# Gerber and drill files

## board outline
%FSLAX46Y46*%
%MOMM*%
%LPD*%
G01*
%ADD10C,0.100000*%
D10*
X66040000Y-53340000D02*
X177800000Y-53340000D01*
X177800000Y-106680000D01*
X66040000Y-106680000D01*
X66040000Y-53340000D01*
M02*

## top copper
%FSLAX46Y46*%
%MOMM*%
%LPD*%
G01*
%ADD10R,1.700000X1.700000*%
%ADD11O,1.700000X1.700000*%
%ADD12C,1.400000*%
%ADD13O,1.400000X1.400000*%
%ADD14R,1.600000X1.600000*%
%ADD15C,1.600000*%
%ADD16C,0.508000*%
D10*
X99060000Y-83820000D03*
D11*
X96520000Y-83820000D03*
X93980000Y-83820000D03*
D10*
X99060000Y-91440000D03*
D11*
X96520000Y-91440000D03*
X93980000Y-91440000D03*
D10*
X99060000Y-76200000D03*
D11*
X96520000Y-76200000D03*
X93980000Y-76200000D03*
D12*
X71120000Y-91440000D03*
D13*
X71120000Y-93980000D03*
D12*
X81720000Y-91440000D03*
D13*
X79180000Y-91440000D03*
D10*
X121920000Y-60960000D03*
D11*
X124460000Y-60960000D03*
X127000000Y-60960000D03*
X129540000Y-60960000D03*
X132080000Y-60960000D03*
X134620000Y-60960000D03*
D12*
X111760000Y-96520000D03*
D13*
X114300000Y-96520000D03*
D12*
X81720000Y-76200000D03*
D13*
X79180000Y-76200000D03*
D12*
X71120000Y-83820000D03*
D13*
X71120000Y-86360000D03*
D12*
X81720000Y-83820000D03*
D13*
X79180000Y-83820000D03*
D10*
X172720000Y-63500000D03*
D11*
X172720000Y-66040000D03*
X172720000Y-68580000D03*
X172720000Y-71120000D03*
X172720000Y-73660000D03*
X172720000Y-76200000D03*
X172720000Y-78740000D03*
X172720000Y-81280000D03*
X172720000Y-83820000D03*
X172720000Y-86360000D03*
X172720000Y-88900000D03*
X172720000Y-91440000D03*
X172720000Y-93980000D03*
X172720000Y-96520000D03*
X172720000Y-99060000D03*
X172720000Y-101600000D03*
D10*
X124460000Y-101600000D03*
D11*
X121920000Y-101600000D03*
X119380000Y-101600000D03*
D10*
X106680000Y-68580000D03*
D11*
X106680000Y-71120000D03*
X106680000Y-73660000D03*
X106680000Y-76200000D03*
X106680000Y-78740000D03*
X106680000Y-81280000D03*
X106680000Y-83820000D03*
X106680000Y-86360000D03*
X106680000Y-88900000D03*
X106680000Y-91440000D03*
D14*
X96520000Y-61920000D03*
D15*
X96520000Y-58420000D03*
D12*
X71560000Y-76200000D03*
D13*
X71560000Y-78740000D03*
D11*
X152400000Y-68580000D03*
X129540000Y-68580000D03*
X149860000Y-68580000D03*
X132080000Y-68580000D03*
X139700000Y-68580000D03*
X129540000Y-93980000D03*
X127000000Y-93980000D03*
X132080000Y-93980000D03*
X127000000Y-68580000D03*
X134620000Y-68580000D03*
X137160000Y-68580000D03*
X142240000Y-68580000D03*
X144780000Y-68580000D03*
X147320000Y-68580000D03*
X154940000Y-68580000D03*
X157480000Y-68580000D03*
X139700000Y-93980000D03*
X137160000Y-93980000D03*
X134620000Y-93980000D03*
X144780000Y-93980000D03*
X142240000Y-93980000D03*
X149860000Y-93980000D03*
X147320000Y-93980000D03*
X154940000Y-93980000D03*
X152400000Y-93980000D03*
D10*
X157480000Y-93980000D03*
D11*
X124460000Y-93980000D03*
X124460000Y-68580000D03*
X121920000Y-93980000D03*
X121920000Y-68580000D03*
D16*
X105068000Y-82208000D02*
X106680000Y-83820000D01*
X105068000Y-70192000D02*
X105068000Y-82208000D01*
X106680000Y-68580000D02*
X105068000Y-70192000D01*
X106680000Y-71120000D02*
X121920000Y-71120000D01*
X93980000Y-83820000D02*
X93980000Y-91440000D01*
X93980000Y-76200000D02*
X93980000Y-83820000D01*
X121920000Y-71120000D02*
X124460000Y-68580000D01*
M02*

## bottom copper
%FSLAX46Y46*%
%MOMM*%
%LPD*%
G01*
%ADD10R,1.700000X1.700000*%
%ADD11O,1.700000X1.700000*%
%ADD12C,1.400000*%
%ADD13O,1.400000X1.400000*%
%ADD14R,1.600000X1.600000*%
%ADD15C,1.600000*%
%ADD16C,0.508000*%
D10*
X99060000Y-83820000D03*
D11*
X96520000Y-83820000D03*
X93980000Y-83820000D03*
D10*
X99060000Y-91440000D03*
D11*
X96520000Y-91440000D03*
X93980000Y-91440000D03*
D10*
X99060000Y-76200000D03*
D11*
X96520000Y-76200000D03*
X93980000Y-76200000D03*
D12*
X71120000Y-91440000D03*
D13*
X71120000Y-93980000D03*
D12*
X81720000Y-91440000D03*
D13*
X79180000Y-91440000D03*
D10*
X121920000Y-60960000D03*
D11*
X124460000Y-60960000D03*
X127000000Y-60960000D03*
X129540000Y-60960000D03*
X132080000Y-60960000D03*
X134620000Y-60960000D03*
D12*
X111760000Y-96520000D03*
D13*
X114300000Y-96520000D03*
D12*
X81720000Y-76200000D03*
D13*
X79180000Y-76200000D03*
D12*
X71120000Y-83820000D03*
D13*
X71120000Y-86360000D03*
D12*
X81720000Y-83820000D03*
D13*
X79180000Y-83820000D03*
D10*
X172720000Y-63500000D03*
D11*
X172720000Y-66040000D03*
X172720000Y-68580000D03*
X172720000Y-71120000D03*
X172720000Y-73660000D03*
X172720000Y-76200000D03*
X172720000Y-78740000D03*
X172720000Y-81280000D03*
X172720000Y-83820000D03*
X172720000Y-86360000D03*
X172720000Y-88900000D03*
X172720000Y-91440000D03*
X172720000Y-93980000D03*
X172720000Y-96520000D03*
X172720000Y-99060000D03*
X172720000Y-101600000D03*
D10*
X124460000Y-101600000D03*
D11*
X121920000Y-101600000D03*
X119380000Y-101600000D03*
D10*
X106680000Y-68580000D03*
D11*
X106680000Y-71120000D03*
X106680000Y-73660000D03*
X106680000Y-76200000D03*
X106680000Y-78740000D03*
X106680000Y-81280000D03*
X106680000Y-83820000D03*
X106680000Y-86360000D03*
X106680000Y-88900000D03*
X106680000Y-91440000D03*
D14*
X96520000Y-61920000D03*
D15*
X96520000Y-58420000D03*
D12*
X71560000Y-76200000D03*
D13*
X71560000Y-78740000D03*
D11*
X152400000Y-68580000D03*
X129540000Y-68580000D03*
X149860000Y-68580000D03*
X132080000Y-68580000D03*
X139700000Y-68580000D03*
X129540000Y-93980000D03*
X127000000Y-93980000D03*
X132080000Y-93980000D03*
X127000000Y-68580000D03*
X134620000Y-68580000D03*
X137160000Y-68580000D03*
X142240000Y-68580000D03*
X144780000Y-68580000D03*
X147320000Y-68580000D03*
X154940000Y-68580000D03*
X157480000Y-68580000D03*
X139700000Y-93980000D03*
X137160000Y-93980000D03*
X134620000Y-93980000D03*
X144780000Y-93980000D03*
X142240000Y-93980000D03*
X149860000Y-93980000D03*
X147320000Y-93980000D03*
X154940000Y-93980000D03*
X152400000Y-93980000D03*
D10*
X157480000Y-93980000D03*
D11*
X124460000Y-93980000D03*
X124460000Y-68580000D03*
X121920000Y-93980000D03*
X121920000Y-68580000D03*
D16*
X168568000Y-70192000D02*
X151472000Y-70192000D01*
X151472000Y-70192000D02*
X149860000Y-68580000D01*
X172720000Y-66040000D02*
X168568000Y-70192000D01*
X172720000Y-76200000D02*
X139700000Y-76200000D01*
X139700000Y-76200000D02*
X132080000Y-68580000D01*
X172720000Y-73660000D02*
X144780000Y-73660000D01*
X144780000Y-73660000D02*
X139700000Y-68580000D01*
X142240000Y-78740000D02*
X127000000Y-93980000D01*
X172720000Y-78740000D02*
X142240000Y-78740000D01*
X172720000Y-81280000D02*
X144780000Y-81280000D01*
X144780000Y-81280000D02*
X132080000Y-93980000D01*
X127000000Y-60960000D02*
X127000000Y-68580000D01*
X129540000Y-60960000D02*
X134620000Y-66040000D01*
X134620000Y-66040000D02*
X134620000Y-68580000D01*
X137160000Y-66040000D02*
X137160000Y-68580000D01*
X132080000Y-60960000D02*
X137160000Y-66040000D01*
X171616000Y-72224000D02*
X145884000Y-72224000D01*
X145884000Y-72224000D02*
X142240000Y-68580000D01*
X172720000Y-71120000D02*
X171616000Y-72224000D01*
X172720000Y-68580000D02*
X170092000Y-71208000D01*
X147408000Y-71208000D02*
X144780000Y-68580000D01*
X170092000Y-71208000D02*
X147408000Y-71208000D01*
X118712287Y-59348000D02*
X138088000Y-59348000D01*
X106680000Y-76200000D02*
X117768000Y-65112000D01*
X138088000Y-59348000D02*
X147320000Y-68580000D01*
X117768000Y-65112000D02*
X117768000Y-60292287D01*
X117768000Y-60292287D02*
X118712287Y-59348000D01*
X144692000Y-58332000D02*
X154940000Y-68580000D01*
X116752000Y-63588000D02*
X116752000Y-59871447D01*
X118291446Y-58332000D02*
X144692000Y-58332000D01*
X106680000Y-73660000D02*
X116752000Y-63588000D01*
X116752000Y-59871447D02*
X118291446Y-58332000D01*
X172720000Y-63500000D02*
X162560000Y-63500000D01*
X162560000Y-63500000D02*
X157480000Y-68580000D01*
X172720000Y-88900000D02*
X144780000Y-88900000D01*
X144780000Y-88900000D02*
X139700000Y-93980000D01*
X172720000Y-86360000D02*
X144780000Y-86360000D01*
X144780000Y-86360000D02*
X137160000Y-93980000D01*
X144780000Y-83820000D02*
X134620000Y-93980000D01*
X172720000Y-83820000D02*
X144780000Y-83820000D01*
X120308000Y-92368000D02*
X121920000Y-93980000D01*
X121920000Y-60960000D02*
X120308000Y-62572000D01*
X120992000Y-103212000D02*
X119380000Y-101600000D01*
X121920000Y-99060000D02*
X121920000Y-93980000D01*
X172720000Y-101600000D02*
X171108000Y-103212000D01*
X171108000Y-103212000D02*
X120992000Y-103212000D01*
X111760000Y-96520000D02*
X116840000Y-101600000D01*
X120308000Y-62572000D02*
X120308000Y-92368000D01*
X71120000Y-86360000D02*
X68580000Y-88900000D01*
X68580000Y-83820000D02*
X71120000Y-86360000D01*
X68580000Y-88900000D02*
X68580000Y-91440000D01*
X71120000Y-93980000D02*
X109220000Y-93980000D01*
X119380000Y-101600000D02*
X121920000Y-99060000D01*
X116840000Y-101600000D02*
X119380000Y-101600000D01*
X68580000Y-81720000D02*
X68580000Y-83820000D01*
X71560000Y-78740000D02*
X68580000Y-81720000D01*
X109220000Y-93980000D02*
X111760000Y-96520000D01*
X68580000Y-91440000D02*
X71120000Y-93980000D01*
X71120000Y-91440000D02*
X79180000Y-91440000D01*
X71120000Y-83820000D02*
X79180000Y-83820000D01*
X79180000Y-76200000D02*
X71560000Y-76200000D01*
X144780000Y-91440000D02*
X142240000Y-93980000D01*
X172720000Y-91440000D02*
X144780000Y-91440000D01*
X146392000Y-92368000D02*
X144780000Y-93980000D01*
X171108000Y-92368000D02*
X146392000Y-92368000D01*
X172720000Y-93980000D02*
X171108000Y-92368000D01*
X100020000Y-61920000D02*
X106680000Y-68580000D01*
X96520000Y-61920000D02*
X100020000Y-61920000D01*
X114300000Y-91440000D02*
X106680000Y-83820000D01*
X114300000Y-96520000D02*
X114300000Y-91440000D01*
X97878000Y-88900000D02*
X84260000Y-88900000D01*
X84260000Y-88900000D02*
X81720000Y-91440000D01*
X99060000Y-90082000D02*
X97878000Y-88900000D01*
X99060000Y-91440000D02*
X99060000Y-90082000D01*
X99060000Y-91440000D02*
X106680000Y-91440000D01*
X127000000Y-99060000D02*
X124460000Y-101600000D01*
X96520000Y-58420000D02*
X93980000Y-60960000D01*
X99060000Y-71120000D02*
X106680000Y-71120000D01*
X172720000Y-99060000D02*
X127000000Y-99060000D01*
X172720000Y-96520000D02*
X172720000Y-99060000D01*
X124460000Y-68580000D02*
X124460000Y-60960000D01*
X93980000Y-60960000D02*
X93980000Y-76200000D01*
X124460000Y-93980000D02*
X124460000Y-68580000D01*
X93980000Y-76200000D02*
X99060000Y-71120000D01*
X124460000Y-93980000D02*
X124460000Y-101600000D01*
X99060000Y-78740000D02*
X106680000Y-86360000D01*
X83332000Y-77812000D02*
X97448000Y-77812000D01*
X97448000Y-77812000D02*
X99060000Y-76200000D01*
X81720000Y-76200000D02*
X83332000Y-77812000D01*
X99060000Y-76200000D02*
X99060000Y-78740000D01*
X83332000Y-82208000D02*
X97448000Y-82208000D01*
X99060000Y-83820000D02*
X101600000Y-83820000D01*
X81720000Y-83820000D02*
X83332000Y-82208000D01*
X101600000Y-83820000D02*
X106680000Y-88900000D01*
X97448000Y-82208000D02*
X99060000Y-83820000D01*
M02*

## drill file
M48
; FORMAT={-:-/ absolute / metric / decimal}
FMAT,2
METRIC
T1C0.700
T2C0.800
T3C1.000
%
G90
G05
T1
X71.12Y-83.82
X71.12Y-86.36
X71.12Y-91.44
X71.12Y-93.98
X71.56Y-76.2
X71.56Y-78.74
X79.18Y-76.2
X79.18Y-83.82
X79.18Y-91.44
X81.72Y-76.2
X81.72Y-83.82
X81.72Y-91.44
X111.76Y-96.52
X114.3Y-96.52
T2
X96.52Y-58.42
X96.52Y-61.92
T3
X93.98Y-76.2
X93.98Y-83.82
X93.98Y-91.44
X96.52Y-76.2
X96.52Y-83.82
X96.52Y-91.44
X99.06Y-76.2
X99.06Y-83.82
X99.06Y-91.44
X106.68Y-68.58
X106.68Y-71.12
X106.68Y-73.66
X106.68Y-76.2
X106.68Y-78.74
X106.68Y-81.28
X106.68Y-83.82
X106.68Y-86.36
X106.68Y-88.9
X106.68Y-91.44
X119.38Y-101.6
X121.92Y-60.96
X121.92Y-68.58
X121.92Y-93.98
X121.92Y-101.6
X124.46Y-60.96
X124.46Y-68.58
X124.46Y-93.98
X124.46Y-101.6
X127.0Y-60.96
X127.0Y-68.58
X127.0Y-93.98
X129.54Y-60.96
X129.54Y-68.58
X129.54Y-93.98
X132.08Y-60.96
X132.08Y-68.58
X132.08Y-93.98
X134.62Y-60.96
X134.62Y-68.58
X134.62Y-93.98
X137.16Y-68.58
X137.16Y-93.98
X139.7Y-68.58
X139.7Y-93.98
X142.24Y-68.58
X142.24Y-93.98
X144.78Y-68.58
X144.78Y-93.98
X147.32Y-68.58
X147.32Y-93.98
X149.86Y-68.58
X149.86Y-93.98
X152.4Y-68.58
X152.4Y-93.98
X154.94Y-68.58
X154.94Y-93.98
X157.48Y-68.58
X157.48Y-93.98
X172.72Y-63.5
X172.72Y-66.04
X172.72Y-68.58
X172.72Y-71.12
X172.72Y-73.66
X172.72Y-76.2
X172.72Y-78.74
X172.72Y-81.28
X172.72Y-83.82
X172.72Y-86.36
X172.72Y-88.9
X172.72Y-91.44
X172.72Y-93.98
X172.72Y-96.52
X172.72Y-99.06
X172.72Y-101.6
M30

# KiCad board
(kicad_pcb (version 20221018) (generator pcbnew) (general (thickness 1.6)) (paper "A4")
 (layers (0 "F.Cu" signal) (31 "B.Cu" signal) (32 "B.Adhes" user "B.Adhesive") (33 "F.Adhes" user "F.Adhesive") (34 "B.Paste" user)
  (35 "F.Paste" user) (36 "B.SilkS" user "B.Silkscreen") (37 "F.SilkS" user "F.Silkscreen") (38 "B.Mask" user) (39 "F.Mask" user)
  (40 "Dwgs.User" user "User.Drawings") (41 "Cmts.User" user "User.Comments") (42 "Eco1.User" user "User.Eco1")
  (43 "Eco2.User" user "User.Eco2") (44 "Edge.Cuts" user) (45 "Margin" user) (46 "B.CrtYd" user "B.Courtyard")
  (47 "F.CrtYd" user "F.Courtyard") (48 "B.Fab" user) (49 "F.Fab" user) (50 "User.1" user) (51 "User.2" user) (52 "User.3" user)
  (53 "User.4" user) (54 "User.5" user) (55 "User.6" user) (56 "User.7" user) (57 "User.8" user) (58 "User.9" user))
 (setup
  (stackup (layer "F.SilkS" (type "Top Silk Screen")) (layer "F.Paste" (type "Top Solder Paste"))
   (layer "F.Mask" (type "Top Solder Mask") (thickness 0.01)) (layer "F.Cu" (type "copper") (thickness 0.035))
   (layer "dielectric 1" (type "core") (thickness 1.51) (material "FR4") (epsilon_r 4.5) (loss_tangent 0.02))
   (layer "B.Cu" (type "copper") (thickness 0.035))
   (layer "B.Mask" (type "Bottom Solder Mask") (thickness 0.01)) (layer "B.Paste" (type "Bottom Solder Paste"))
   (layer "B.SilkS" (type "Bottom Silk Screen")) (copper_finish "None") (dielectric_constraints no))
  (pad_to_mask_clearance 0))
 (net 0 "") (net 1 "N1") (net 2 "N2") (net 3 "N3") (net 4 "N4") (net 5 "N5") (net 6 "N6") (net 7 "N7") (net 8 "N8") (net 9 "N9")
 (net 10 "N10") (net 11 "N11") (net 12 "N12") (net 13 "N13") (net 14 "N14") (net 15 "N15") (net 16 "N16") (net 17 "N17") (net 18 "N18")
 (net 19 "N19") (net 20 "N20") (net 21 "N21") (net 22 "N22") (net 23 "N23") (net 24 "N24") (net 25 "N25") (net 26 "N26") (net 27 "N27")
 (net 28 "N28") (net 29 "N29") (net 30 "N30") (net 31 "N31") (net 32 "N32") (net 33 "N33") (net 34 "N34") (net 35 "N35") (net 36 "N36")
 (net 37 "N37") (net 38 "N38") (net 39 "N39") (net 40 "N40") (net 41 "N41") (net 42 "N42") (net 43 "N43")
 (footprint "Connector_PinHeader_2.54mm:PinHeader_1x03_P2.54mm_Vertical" (layer "F.Cu") (at 99.06 83.82 -90)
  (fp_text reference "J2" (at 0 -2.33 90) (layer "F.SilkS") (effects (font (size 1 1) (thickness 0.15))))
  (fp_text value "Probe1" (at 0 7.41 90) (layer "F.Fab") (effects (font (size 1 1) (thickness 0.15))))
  (pad "1" thru_hole rect (at 0 0 270) (size 1.7 1.7) (drill 1) (layers "*.Cu" "*.Mask") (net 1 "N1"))
  (pad "2" thru_hole oval (at 0 2.54 270) (size 1.7 1.7) (drill 1) (layers "*.Cu" "*.Mask") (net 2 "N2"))
  (pad "3" thru_hole oval (at 0 5.08 270) (size 1.7 1.7) (drill 1) (layers "*.Cu" "*.Mask") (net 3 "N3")))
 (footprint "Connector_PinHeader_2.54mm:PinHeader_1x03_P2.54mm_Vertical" (layer "F.Cu") (at 99.06 91.44 -90)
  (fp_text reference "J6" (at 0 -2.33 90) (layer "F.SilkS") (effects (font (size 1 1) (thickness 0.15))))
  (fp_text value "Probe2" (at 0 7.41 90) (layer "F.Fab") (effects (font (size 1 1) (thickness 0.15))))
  (pad "1" thru_hole rect (at 0 0 270) (size 1.7 1.7) (drill 1) (layers "*.Cu" "*.Mask") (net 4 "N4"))
  (pad "2" thru_hole oval (at 0 2.54 270) (size 1.7 1.7) (drill 1) (layers "*.Cu" "*.Mask") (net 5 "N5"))
  (pad "3" thru_hole oval (at 0 5.08 270) (size 1.7 1.7) (drill 1) (layers "*.Cu" "*.Mask") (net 3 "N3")))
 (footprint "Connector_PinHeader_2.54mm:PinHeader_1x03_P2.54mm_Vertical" (layer "F.Cu") (at 99.06 76.2 -90)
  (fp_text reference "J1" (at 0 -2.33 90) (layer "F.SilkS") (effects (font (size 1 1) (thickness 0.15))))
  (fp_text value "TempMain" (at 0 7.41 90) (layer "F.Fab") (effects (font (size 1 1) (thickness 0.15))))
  (pad "1" thru_hole rect (at 0 0 270) (size 1.7 1.7) (drill 1) (layers "*.Cu" "*.Mask") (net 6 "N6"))
  (pad "2" thru_hole oval (at 0 2.54 270) (size 1.7 1.7) (drill 1) (layers "*.Cu" "*.Mask") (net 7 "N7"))
  (pad "3" thru_hole oval (at 0 5.08 270) (size 1.7 1.7) (drill 1) (layers "*.Cu" "*.Mask") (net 3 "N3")))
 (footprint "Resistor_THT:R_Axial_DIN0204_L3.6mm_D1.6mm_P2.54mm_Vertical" (layer "F.Cu") (at 71.12 91.44 -90)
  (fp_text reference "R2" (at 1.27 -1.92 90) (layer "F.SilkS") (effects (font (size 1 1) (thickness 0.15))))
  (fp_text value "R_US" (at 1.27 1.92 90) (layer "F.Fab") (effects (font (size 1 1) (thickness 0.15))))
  (pad "1" thru_hole circle (at 0 0 270) (size 1.4 1.4) (drill 0.7) (layers "*.Cu" "*.Mask") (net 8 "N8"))
  (pad "2" thru_hole oval (at 2.54 0 270) (size 1.4 1.4) (drill 0.7) (layers "*.Cu" "*.Mask") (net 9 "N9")))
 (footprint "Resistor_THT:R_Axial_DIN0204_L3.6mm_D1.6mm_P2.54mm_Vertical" (layer "F.Cu") (at 81.72 91.44 180)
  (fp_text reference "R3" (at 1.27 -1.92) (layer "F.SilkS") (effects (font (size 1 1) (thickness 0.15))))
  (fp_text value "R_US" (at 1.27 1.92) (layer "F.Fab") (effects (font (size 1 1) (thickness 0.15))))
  (pad "1" thru_hole circle (at 0 0 180) (size 1.4 1.4) (drill 0.7) (layers "*.Cu" "*.Mask") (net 4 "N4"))
  (pad "2" thru_hole oval (at 2.54 0 180) (size 1.4 1.4) (drill 0.7) (layers "*.Cu" "*.Mask") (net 8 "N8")))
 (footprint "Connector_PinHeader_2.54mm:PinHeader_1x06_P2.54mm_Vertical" (layer "F.Cu") (at 121.92 60.96 90)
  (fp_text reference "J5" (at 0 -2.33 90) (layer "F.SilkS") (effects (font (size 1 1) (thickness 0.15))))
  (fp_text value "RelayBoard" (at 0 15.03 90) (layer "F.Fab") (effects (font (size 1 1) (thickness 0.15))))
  (pad "1" thru_hole rect (at 0 0 90) (size 1.7 1.7) (drill 1) (layers "*.Cu" "*.Mask") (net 9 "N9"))
  (pad "2" thru_hole oval (at 0 2.54 90) (size 1.7 1.7) (drill 1) (layers "*.Cu" "*.Mask") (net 3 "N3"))
  (pad "3" thru_hole oval (at 0 5.08 90) (size 1.7 1.7) (drill 1) (layers "*.Cu" "*.Mask") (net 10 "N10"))
  (pad "4" thru_hole oval (at 0 7.62 90) (size 1.7 1.7) (drill 1) (layers "*.Cu" "*.Mask") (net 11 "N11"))
  (pad "5" thru_hole oval (at 0 10.16 90) (size 1.7 1.7) (drill 1) (layers "*.Cu" "*.Mask") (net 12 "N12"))
  (pad "6" thru_hole oval (at 0 12.7 90) (size 1.7 1.7) (drill 1) (layers "*.Cu" "*.Mask") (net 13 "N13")))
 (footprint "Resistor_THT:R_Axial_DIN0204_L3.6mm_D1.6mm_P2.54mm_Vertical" (layer "F.Cu") (at 111.76 96.52)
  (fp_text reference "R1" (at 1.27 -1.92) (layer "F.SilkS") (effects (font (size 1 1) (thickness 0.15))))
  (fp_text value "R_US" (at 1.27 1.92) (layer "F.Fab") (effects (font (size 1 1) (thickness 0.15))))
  (pad "1" thru_hole circle (at 0 0) (size 1.4 1.4) (drill 0.7) (layers "*.Cu" "*.Mask") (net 9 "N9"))
  (pad "2" thru_hole oval (at 2.54 0) (size 1.4 1.4) (drill 0.7) (layers "*.Cu" "*.Mask") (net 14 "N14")))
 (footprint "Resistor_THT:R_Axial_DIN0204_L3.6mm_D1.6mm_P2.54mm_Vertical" (layer "F.Cu") (at 81.72 76.2 180)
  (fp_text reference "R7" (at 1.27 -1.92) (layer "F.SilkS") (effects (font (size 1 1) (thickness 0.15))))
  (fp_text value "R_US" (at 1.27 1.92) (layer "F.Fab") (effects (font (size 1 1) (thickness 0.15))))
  (pad "1" thru_hole circle (at 0 0 180) (size 1.4 1.4) (drill 0.7) (layers "*.Cu" "*.Mask") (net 6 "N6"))
  (pad "2" thru_hole oval (at 2.54 0 180) (size 1.4 1.4) (drill 0.7) (layers "*.Cu" "*.Mask") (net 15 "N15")))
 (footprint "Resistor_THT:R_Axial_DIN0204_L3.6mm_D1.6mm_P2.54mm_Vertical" (layer "F.Cu") (at 71.12 83.82 -90)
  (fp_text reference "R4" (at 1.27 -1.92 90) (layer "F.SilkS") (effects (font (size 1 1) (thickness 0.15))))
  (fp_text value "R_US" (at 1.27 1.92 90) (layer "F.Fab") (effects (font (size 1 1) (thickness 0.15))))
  (pad "1" thru_hole circle (at 0 0 270) (size 1.4 1.4) (drill 0.7) (layers "*.Cu" "*.Mask") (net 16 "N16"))
  (pad "2" thru_hole oval (at 2.54 0 270) (size 1.4 1.4) (drill 0.7) (layers "*.Cu" "*.Mask") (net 9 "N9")))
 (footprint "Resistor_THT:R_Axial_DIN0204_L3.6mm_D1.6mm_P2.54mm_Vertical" (layer "F.Cu") (at 81.72 83.82 180)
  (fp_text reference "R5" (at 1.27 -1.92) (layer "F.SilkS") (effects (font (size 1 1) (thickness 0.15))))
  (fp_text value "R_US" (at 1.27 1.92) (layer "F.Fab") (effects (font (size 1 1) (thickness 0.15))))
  (pad "1" thru_hole circle (at 0 0 180) (size 1.4 1.4) (drill 0.7) (layers "*.Cu" "*.Mask") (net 1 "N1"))
  (pad "2" thru_hole oval (at 2.54 0 180) (size 1.4 1.4) (drill 0.7) (layers "*.Cu" "*.Mask") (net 16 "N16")))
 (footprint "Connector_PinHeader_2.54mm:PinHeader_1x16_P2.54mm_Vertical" (layer "F.Cu") (at 172.72 63.5)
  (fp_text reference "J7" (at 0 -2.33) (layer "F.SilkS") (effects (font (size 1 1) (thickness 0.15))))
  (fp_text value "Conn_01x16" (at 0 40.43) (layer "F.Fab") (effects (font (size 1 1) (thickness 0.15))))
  (pad "1" thru_hole rect (at 0 0) (size 1.7 1.7) (drill 1) (layers "*.Cu" "*.Mask") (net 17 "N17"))
  (pad "2" thru_hole oval (at 0 2.54) (size 1.7 1.7) (drill 1) (layers "*.Cu" "*.Mask") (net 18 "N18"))
  (pad "3" thru_hole oval (at 0 5.08) (size 1.7 1.7) (drill 1) (layers "*.Cu" "*.Mask") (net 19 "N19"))
  (pad "4" thru_hole oval (at 0 7.62) (size 1.7 1.7) (drill 1) (layers "*.Cu" "*.Mask") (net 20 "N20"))
  (pad "5" thru_hole oval (at 0 10.16) (size 1.7 1.7) (drill 1) (layers "*.Cu" "*.Mask") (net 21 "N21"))
  (pad "6" thru_hole oval (at 0 12.7) (size 1.7 1.7) (drill 1) (layers "*.Cu" "*.Mask") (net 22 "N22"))
  (pad "7" thru_hole oval (at 0 15.24) (size 1.7 1.7) (drill 1) (layers "*.Cu" "*.Mask") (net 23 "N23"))
  (pad "8" thru_hole oval (at 0 17.78) (size 1.7 1.7) (drill 1) (layers "*.Cu" "*.Mask") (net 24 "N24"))
  (pad "9" thru_hole oval (at 0 20.32) (size 1.7 1.7) (drill 1) (layers "*.Cu" "*.Mask") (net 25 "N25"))
  (pad "10" thru_hole oval (at 0 22.86) (size 1.7 1.7) (drill 1) (layers "*.Cu" "*.Mask") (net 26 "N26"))
  (pad "11" thru_hole oval (at 0 25.4) (size 1.7 1.7) (drill 1) (layers "*.Cu" "*.Mask") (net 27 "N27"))
  (pad "12" thru_hole oval (at 0 27.94) (size 1.7 1.7) (drill 1) (layers "*.Cu" "*.Mask") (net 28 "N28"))
  (pad "13" thru_hole oval (at 0 30.48) (size 1.7 1.7) (drill 1) (layers "*.Cu" "*.Mask") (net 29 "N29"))
  (pad "14" thru_hole oval (at 0 33.02) (size 1.7 1.7) (drill 1) (layers "*.Cu" "*.Mask") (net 3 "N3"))
  (pad "15" thru_hole oval (at 0 35.56) (size 1.7 1.7) (drill 1) (layers "*.Cu" "*.Mask") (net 3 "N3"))
  (pad "16" thru_hole oval (at 0 38.1) (size 1.7 1.7) (drill 1) (layers "*.Cu" "*.Mask") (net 9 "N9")))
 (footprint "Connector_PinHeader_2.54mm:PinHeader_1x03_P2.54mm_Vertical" (layer "F.Cu") (at 124.46 101.6 -90)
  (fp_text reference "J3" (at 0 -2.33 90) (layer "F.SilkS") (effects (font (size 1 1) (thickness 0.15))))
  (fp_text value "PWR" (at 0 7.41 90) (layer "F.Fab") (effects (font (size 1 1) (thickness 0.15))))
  (pad "1" thru_hole rect (at 0 0 270) (size 1.7 1.7) (drill 1) (layers "*.Cu" "*.Mask") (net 3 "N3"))
  (pad "2" thru_hole oval (at 0 2.54 270) (size 1.7 1.7) (drill 1) (layers "*.Cu" "*.Mask") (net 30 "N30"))
  (pad "3" thru_hole oval (at 0 5.08 270) (size 1.7 1.7) (drill 1) (layers "*.Cu" "*.Mask") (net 9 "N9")))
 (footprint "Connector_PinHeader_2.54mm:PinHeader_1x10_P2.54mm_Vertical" (layer "F.Cu") (at 106.68 68.58)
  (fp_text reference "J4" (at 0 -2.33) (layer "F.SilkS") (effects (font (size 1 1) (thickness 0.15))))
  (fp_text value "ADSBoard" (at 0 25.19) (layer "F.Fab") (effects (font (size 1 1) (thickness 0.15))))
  (pad "1" thru_hole rect (at 0 0) (size 1.7 1.7) (drill 1) (layers "*.Cu" "*.Mask") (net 14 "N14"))
  (pad "2" thru_hole oval (at 0 2.54) (size 1.7 1.7) (drill 1) (layers "*.Cu" "*.Mask") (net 3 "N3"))
  (pad "3" thru_hole oval (at 0 5.08) (size 1.7 1.7) (drill 1) (layers "*.Cu" "*.Mask") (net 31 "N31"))
  (pad "4" thru_hole oval (at 0 7.62) (size 1.7 1.7) (drill 1) (layers "*.Cu" "*.Mask") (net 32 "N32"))
  (pad "5" thru_hole oval (at 0 10.16) (size 1.7 1.7) (drill 1) (layers "*.Cu" "*.Mask") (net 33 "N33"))
  (pad "6" thru_hole oval (at 0 12.7) (size 1.7 1.7) (drill 1) (layers "*.Cu" "*.Mask") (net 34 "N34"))
  (pad "7" thru_hole oval (at 0 15.24) (size 1.7 1.7) (drill 1) (layers "*.Cu" "*.Mask") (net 14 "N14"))
  (pad "8" thru_hole oval (at 0 17.78) (size 1.7 1.7) (drill 1) (layers "*.Cu" "*.Mask") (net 6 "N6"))
  (pad "9" thru_hole oval (at 0 20.32) (size 1.7 1.7) (drill 1) (layers "*.Cu" "*.Mask") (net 1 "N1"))
  (pad "10" thru_hole oval (at 0 22.86) (size 1.7 1.7) (drill 1) (layers "*.Cu" "*.Mask") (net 4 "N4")))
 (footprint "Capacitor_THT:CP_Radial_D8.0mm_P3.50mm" (layer "F.Cu") (at 96.52 61.92 90)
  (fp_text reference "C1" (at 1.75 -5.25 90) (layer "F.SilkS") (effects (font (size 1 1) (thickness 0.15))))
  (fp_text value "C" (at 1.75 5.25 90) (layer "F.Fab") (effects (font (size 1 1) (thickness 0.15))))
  (pad "1" thru_hole rect (at 0 0 90) (size 1.6 1.6) (drill 0.8) (layers "*.Cu" "*.Mask") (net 14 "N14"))
  (pad "2" thru_hole circle (at 3.5 0 90) (size 1.6 1.6) (drill 0.8) (layers "*.Cu" "*.Mask") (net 3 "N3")))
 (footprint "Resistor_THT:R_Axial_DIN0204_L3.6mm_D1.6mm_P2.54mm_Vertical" (layer "F.Cu") (at 71.56 76.2 -90)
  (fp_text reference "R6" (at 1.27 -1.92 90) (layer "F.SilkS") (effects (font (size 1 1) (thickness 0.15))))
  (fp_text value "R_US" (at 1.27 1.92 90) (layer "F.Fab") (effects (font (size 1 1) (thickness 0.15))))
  (pad "1" thru_hole circle (at 0 0 270) (size 1.4 1.4) (drill 0.7) (layers "*.Cu" "*.Mask") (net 15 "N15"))
  (pad "2" thru_hole oval (at 2.54 0 270) (size 1.4 1.4) (drill 0.7) (layers "*.Cu" "*.Mask") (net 9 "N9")))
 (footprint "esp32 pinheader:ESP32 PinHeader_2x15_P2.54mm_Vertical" (layer "B.Cu") (at 157.48 93.98 90)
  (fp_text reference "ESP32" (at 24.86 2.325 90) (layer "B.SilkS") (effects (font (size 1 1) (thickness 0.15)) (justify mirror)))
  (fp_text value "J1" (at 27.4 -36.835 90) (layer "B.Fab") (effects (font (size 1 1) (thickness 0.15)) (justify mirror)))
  (pad "1" thru_hole oval (at 25.4 -5.08 90) (size 1.7 1.7) (drill 1) (layers "*.Cu" "*.Mask") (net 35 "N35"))
  (pad "2" thru_hole oval (at 25.4 -27.94 90) (size 1.7 1.7) (drill 1) (layers "*.Cu" "*.Mask") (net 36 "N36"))
  (pad "3" thru_hole oval (at 25.4 -7.62 90) (size 1.7 1.7) (drill 1) (layers "*.Cu" "*.Mask") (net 18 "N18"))
  (pad "4" thru_hole oval (at 25.4 -25.4 90) (size 1.7 1.7) (drill 1) (layers "*.Cu" "*.Mask") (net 22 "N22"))
  (pad "5" thru_hole oval (at 25.4 -17.78 90) (size 1.7 1.7) (drill 1) (layers "*.Cu" "*.Mask") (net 21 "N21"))
  (pad "12" thru_hole oval (at 0 -27.94 90) (size 1.7 1.7) (drill 1) (layers "*.Cu" "*.Mask") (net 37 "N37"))
  (pad "13" thru_hole oval (at 0 -30.48 90) (size 1.7 1.7) (drill 1) (layers "*.Cu" "*.Mask") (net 23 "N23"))
  (pad "14" thru_hole oval (at 0 -25.4 90) (size 1.7 1.7) (drill 1) (layers "*.Cu" "*.Mask") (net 24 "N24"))
  (pad "15" thru_hole oval (at 25.4 -30.48 90) (size 1.7 1.7) (drill 1) (layers "*.Cu" "*.Mask") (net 10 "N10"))
  (pad "16" thru_hole oval (at 25.4 -22.86 90) (size 1.7 1.7) (drill 1) (layers "*.Cu" "*.Mask") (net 11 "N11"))
  (pad "17" thru_hole oval (at 25.4 -20.32 90) (size 1.7 1.7) (drill 1) (layers "*.Cu" "*.Mask") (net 12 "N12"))
  (pad "18" thru_hole oval (at 25.4 -15.24 90) (size 1.7 1.7) (drill 1) (layers "*.Cu" "*.Mask") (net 20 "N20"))
  (pad "19" thru_hole oval (at 25.4 -12.7 90) (size 1.7 1.7) (drill 1) (layers "*.Cu" "*.Mask") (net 19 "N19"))
  (pad "21" thru_hole oval (at 25.4 -10.16 90) (size 1.7 1.7) (drill 1) (layers "*.Cu" "*.Mask") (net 32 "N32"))
  (pad "22" thru_hole oval (at 25.4 -2.54 90) (size 1.7 1.7) (drill 1) (layers "*.Cu" "*.Mask") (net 31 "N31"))
  (pad "23" thru_hole oval (at 25.4 0 90) (size 1.7 1.7) (drill 1) (layers "*.Cu" "*.Mask") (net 17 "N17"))
  (pad "25" thru_hole oval (at 0 -17.78 90) (size 1.7 1.7) (drill 1) (layers "*.Cu" "*.Mask") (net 27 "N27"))
  (pad "26" thru_hole oval (at 0 -20.32 90) (size 1.7 1.7) (drill 1) (layers "*.Cu" "*.Mask") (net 26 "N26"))
  (pad "27" thru_hole oval (at 0 -22.86 90) (size 1.7 1.7) (drill 1) (layers "*.Cu" "*.Mask") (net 25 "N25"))
  (pad "32" thru_hole oval (at 0 -12.7 90) (size 1.7 1.7) (drill 1) (layers "*.Cu" "*.Mask") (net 29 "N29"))
  (pad "33" thru_hole oval (at 0 -15.24 90) (size 1.7 1.7) (drill 1) (layers "*.Cu" "*.Mask") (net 28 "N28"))
  (pad "34" thru_hole oval (at 0 -7.62 90) (size 1.7 1.7) (drill 1) (layers "*.Cu" "*.Mask") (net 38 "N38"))
  (pad "35" thru_hole oval (at 0 -10.16 90) (size 1.7 1.7) (drill 1) (layers "*.Cu" "*.Mask") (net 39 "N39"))
  (pad "36" thru_hole oval (at 0 -2.54 90) (size 1.7 1.7) (drill 1) (layers "*.Cu" "*.Mask") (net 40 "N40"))
  (pad "39" thru_hole oval (at 0 -5.08 90) (size 1.7 1.7) (drill 1) (layers "*.Cu" "*.Mask") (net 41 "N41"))
  (pad "60" thru_hole rect (at 0 0 90) (size 1.7 1.7) (drill 1) (layers "*.Cu" "*.Mask") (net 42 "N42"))
  (pad "61" thru_hole oval (at 0 -33.02 90) (size 1.7 1.7) (drill 1) (layers "*.Cu" "*.Mask") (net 3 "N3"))
  (pad "62" thru_hole oval (at 25.4 -33.02 90) (size 1.7 1.7) (drill 1) (layers "*.Cu" "*.Mask") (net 3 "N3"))
  (pad "63" thru_hole oval (at 0 -35.56 90) (size 1.7 1.7) (drill 1) (layers "*.Cu" "*.Mask") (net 9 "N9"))
  (pad "64" thru_hole oval (at 25.4 -35.56 90) (size 1.7 1.7) (drill 1) (layers "*.Cu" "*.Mask") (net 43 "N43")))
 (gr_rect (start 66.04 53.34) (end 177.8 106.68) (stroke (width 0.1) (type default)) (fill none) (layer "Edge.Cuts"))
 (segment (start 168.568 70.192) (end 151.472 70.192) (width 0.508) (layer "B.Cu") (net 18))
 (segment (start 151.472 70.192) (end 149.86 68.58) (width 0.508) (layer "B.Cu") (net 18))
 (segment (start 172.72 66.04) (end 168.568 70.192) (width 0.508) (layer "B.Cu") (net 18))
 (segment (start 172.72 76.2) (end 139.7 76.2) (width 0.508) (layer "B.Cu") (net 22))
 (segment (start 139.7 76.2) (end 132.08 68.58) (width 0.508) (layer "B.Cu") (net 22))
 (segment (start 172.72 73.66) (end 144.78 73.66) (width 0.508) (layer "B.Cu") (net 21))
 (segment (start 144.78 73.66) (end 139.7 68.58) (width 0.508) (layer "B.Cu") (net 21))
 (segment (start 142.24 78.74) (end 127 93.98) (width 0.508) (layer "B.Cu") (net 23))
 (segment (start 172.72 78.74) (end 142.24 78.74) (width 0.508) (layer "B.Cu") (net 23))
 (segment (start 172.72 81.28) (end 144.78 81.28) (width 0.508) (layer "B.Cu") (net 24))
 (segment (start 144.78 81.28) (end 132.08 93.98) (width 0.508) (layer "B.Cu") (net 24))
 (segment (start 127 60.96) (end 127 68.58) (width 0.508) (layer "B.Cu") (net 10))
 (segment (start 129.54 60.96) (end 134.62 66.04) (width 0.508) (layer "B.Cu") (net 11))
 (segment (start 134.62 66.04) (end 134.62 68.58) (width 0.508) (layer "B.Cu") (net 11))
 (segment (start 137.16 66.04) (end 137.16 68.58) (width 0.508) (layer "B.Cu") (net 12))
 (segment (start 132.08 60.96) (end 137.16 66.04) (width 0.508) (layer "B.Cu") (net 12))
 (segment (start 171.616 72.224) (end 145.884 72.224) (width 0.508) (layer "B.Cu") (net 20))
 (segment (start 145.884 72.224) (end 142.24 68.58) (width 0.508) (layer "B.Cu") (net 20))
 (segment (start 172.72 71.12) (end 171.616 72.224) (width 0.508) (layer "B.Cu") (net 20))
 (segment (start 172.72 68.58) (end 170.092 71.208) (width 0.508) (layer "B.Cu") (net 19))
 (segment (start 147.408 71.208) (end 144.78 68.58) (width 0.508) (layer "B.Cu") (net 19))
 (segment (start 170.092 71.208) (end 147.408 71.208) (width 0.508) (layer "B.Cu") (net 19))
 (segment (start 118.712287 59.348) (end 138.088 59.348) (width 0.508) (layer "B.Cu") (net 32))
 (segment (start 106.68 76.2) (end 117.768 65.112) (width 0.508) (layer "B.Cu") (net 32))
 (segment (start 138.088 59.348) (end 147.32 68.58) (width 0.508) (layer "B.Cu") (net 32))
 (segment (start 117.768 65.112) (end 117.768 60.292287) (width 0.508) (layer "B.Cu") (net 32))
 (segment (start 117.768 60.292287) (end 118.712287 59.348) (width 0.508) (layer "B.Cu") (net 32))
 (segment (start 144.692 58.332) (end 154.94 68.58) (width 0.508) (layer "B.Cu") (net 31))
 (segment (start 116.752 63.588) (end 116.752 59.871447) (width 0.508) (layer "B.Cu") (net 31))
 (segment (start 118.291446 58.332) (end 144.692 58.332) (width 0.508) (layer "B.Cu") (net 31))
 (segment (start 106.68 73.66) (end 116.752 63.588) (width 0.508) (layer "B.Cu") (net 31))
 (segment (start 116.752 59.871447) (end 118.291446 58.332) (width 0.508) (layer "B.Cu") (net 31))
 (segment (start 172.72 63.5) (end 162.56 63.5) (width 0.508) (layer "B.Cu") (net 17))
 (segment (start 162.56 63.5) (end 157.48 68.58) (width 0.508) (layer "B.Cu") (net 17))
 (segment (start 172.72 88.9) (end 144.78 88.9) (width 0.508) (layer "B.Cu") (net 27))
 (segment (start 144.78 88.9) (end 139.7 93.98) (width 0.508) (layer "B.Cu") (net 27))
 (segment (start 172.72 86.36) (end 144.78 86.36) (width 0.508) (layer "B.Cu") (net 26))
 (segment (start 144.78 86.36) (end 137.16 93.98) (width 0.508) (layer "B.Cu") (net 26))
 (segment (start 144.78 83.82) (end 134.62 93.98) (width 0.508) (layer "B.Cu") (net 25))
 (segment (start 172.72 83.82) (end 144.78 83.82) (width 0.508) (layer "B.Cu") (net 25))
 (segment (start 120.308 92.368) (end 121.92 93.98) (width 0.508) (layer "B.Cu") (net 9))
 (segment (start 121.92 60.96) (end 120.308 62.572) (width 0.508) (layer "B.Cu") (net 9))
 (segment (start 120.992 103.212) (end 119.38 101.6) (width 0.508) (layer "B.Cu") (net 9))
 (segment (start 121.92 99.06) (end 121.92 93.98) (width 0.508) (layer "B.Cu") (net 9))
 (segment (start 172.72 101.6) (end 171.108 103.212) (width 0.508) (layer "B.Cu") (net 9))
 (segment (start 171.108 103.212) (end 120.992 103.212) (width 0.508) (layer "B.Cu") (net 9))
 (segment (start 111.76 96.52) (end 116.84 101.6) (width 0.508) (layer "B.Cu") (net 9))
 (segment (start 120.308 62.572) (end 120.308 92.368) (width 0.508) (layer "B.Cu") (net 9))
 (segment (start 71.12 86.36) (end 68.58 88.9) (width 0.508) (layer "B.Cu") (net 9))
 (segment (start 68.58 83.82) (end 71.12 86.36) (width 0.508) (layer "B.Cu") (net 9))
 (segment (start 68.58 88.9) (end 68.58 91.44) (width 0.508) (layer "B.Cu") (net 9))
 (segment (start 71.12 93.98) (end 109.22 93.98) (width 0.508) (layer "B.Cu") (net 9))
 (segment (start 119.38 101.6) (end 121.92 99.06) (width 0.508) (layer "B.Cu") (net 9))
 (segment (start 116.84 101.6) (end 119.38 101.6) (width 0.508) (layer "B.Cu") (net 9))
 (segment (start 68.58 81.72) (end 68.58 83.82) (width 0.508) (layer "B.Cu") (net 9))
 (segment (start 71.56 78.74) (end 68.58 81.72) (width 0.508) (layer "B.Cu") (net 9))
 (segment (start 109.22 93.98) (end 111.76 96.52) (width 0.508) (layer "B.Cu") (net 9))
 (segment (start 68.58 91.44) (end 71.12 93.98) (width 0.508) (layer "B.Cu") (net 9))
 (segment (start 71.12 91.44) (end 79.18 91.44) (width 0.508) (layer "B.Cu") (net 8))
 (segment (start 71.12 83.82) (end 79.18 83.82) (width 0.508) (layer "B.Cu") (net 16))
 (segment (start 79.18 76.2) (end 71.56 76.2) (width 0.508) (layer "B.Cu") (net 15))
 (segment (start 144.78 91.44) (end 142.24 93.98) (width 0.508) (layer "B.Cu") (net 28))
 (segment (start 172.72 91.44) (end 144.78 91.44) (width 0.508) (layer "B.Cu") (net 28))
 (segment (start 146.392 92.368) (end 144.78 93.98) (width 0.508) (layer "B.Cu") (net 29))
 (segment (start 171.108 92.368) (end 146.392 92.368) (width 0.508) (layer "B.Cu") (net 29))
 (segment (start 172.72 93.98) (end 171.108 92.368) (width 0.508) (layer "B.Cu") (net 29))
 (segment (start 105.068 82.208) (end 106.68 83.82) (width 0.508) (layer "F.Cu") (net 14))
 (segment (start 105.068 70.192) (end 105.068 82.208) (width 0.508) (layer "F.Cu") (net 14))
 (segment (start 106.68 68.58) (end 105.068 70.192) (width 0.508) (layer "F.Cu") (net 14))
 (segment (start 100.02 61.92) (end 106.68 68.58) (width 0.508) (layer "B.Cu") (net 14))
 (segment (start 96.52 61.92) (end 100.02 61.92) (width 0.508) (layer "B.Cu") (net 14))
 (segment (start 114.3 91.44) (end 106.68 83.82) (width 0.508) (layer "B.Cu") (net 14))
 (segment (start 114.3 96.52) (end 114.3 91.44) (width 0.508) (layer "B.Cu") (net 14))
 (segment (start 97.878 88.9) (end 84.26 88.9) (width 0.508) (layer "B.Cu") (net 4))
 (segment (start 84.26 88.9) (end 81.72 91.44) (width 0.508) (layer "B.Cu") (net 4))
 (segment (start 99.06 90.082) (end 97.878 88.9) (width 0.508) (layer "B.Cu") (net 4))
 (segment (start 99.06 91.44) (end 99.06 90.082) (width 0.508) (layer "B.Cu") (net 4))
 (segment (start 99.06 91.44) (end 106.68 91.44) (width 0.508) (layer "B.Cu") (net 4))
 (segment (start 106.68 71.12) (end 121.92 71.12) (width 0.508) (layer "F.Cu") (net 3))
 (segment (start 93.98 83.82) (end 93.98 91.44) (width 0.508) (layer "F.Cu") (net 3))
 (segment (start 93.98 76.2) (end 93.98 83.82) (width 0.508) (layer "F.Cu") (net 3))
 (segment (start 121.92 71.12) (end 124.46 68.58) (width 0.508) (layer "F.Cu") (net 3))
 (segment (start 127 99.06) (end 124.46 101.6) (width 0.508) (layer "B.Cu") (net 3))
 (segment (start 96.52 58.42) (end 93.98 60.96) (width 0.508) (layer "B.Cu") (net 3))
 (segment (start 99.06 71.12) (end 106.68 71.12) (width 0.508) (layer "B.Cu") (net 3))
 (segment (start 172.72 99.06) (end 127 99.06) (width 0.508) (layer "B.Cu") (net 3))
 (segment (start 172.72 96.52) (end 172.72 99.06) (width 0.508) (layer "B.Cu") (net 3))
 (segment (start 124.46 68.58) (end 124.46 60.96) (width 0.508) (layer "B.Cu") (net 3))
 (segment (start 93.98 60.96) (end 93.98 76.2) (width 0.508) (layer "B.Cu") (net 3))
 (segment (start 124.46 93.98) (end 124.46 68.58) (width 0.508) (layer "B.Cu") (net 3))
 (segment (start 93.98 76.2) (end 99.06 71.12) (width 0.508) (layer "B.Cu") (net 3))
 (segment (start 124.46 93.98) (end 124.46 101.6) (width 0.508) (layer "B.Cu") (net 3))
 (segment (start 99.06 78.74) (end 106.68 86.36) (width 0.508) (layer "B.Cu") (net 6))
 (segment (start 83.332 77.812) (end 97.448 77.812) (width 0.508) (layer "B.Cu") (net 6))
 (segment (start 97.448 77.812) (end 99.06 76.2) (width 0.508) (layer "B.Cu") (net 6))
 (segment (start 81.72 76.2) (end 83.332 77.812) (width 0.508) (layer "B.Cu") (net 6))
 (segment (start 99.06 76.2) (end 99.06 78.74) (width 0.508) (layer "B.Cu") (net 6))
 (segment (start 83.332 82.208) (end 97.448 82.208) (width 0.508) (layer "B.Cu") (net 1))
 (segment (start 99.06 83.82) (end 101.6 83.82) (width 0.508) (layer "B.Cu") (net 1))
 (segment (start 81.72 83.82) (end 83.332 82.208) (width 0.508) (layer "B.Cu") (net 1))
 (segment (start 101.6 83.82) (end 106.68 88.9) (width 0.508) (layer "B.Cu") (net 1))
 (segment (start 97.448 82.208) (end 99.06 83.82) (width 0.508) (layer "B.Cu") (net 1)))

